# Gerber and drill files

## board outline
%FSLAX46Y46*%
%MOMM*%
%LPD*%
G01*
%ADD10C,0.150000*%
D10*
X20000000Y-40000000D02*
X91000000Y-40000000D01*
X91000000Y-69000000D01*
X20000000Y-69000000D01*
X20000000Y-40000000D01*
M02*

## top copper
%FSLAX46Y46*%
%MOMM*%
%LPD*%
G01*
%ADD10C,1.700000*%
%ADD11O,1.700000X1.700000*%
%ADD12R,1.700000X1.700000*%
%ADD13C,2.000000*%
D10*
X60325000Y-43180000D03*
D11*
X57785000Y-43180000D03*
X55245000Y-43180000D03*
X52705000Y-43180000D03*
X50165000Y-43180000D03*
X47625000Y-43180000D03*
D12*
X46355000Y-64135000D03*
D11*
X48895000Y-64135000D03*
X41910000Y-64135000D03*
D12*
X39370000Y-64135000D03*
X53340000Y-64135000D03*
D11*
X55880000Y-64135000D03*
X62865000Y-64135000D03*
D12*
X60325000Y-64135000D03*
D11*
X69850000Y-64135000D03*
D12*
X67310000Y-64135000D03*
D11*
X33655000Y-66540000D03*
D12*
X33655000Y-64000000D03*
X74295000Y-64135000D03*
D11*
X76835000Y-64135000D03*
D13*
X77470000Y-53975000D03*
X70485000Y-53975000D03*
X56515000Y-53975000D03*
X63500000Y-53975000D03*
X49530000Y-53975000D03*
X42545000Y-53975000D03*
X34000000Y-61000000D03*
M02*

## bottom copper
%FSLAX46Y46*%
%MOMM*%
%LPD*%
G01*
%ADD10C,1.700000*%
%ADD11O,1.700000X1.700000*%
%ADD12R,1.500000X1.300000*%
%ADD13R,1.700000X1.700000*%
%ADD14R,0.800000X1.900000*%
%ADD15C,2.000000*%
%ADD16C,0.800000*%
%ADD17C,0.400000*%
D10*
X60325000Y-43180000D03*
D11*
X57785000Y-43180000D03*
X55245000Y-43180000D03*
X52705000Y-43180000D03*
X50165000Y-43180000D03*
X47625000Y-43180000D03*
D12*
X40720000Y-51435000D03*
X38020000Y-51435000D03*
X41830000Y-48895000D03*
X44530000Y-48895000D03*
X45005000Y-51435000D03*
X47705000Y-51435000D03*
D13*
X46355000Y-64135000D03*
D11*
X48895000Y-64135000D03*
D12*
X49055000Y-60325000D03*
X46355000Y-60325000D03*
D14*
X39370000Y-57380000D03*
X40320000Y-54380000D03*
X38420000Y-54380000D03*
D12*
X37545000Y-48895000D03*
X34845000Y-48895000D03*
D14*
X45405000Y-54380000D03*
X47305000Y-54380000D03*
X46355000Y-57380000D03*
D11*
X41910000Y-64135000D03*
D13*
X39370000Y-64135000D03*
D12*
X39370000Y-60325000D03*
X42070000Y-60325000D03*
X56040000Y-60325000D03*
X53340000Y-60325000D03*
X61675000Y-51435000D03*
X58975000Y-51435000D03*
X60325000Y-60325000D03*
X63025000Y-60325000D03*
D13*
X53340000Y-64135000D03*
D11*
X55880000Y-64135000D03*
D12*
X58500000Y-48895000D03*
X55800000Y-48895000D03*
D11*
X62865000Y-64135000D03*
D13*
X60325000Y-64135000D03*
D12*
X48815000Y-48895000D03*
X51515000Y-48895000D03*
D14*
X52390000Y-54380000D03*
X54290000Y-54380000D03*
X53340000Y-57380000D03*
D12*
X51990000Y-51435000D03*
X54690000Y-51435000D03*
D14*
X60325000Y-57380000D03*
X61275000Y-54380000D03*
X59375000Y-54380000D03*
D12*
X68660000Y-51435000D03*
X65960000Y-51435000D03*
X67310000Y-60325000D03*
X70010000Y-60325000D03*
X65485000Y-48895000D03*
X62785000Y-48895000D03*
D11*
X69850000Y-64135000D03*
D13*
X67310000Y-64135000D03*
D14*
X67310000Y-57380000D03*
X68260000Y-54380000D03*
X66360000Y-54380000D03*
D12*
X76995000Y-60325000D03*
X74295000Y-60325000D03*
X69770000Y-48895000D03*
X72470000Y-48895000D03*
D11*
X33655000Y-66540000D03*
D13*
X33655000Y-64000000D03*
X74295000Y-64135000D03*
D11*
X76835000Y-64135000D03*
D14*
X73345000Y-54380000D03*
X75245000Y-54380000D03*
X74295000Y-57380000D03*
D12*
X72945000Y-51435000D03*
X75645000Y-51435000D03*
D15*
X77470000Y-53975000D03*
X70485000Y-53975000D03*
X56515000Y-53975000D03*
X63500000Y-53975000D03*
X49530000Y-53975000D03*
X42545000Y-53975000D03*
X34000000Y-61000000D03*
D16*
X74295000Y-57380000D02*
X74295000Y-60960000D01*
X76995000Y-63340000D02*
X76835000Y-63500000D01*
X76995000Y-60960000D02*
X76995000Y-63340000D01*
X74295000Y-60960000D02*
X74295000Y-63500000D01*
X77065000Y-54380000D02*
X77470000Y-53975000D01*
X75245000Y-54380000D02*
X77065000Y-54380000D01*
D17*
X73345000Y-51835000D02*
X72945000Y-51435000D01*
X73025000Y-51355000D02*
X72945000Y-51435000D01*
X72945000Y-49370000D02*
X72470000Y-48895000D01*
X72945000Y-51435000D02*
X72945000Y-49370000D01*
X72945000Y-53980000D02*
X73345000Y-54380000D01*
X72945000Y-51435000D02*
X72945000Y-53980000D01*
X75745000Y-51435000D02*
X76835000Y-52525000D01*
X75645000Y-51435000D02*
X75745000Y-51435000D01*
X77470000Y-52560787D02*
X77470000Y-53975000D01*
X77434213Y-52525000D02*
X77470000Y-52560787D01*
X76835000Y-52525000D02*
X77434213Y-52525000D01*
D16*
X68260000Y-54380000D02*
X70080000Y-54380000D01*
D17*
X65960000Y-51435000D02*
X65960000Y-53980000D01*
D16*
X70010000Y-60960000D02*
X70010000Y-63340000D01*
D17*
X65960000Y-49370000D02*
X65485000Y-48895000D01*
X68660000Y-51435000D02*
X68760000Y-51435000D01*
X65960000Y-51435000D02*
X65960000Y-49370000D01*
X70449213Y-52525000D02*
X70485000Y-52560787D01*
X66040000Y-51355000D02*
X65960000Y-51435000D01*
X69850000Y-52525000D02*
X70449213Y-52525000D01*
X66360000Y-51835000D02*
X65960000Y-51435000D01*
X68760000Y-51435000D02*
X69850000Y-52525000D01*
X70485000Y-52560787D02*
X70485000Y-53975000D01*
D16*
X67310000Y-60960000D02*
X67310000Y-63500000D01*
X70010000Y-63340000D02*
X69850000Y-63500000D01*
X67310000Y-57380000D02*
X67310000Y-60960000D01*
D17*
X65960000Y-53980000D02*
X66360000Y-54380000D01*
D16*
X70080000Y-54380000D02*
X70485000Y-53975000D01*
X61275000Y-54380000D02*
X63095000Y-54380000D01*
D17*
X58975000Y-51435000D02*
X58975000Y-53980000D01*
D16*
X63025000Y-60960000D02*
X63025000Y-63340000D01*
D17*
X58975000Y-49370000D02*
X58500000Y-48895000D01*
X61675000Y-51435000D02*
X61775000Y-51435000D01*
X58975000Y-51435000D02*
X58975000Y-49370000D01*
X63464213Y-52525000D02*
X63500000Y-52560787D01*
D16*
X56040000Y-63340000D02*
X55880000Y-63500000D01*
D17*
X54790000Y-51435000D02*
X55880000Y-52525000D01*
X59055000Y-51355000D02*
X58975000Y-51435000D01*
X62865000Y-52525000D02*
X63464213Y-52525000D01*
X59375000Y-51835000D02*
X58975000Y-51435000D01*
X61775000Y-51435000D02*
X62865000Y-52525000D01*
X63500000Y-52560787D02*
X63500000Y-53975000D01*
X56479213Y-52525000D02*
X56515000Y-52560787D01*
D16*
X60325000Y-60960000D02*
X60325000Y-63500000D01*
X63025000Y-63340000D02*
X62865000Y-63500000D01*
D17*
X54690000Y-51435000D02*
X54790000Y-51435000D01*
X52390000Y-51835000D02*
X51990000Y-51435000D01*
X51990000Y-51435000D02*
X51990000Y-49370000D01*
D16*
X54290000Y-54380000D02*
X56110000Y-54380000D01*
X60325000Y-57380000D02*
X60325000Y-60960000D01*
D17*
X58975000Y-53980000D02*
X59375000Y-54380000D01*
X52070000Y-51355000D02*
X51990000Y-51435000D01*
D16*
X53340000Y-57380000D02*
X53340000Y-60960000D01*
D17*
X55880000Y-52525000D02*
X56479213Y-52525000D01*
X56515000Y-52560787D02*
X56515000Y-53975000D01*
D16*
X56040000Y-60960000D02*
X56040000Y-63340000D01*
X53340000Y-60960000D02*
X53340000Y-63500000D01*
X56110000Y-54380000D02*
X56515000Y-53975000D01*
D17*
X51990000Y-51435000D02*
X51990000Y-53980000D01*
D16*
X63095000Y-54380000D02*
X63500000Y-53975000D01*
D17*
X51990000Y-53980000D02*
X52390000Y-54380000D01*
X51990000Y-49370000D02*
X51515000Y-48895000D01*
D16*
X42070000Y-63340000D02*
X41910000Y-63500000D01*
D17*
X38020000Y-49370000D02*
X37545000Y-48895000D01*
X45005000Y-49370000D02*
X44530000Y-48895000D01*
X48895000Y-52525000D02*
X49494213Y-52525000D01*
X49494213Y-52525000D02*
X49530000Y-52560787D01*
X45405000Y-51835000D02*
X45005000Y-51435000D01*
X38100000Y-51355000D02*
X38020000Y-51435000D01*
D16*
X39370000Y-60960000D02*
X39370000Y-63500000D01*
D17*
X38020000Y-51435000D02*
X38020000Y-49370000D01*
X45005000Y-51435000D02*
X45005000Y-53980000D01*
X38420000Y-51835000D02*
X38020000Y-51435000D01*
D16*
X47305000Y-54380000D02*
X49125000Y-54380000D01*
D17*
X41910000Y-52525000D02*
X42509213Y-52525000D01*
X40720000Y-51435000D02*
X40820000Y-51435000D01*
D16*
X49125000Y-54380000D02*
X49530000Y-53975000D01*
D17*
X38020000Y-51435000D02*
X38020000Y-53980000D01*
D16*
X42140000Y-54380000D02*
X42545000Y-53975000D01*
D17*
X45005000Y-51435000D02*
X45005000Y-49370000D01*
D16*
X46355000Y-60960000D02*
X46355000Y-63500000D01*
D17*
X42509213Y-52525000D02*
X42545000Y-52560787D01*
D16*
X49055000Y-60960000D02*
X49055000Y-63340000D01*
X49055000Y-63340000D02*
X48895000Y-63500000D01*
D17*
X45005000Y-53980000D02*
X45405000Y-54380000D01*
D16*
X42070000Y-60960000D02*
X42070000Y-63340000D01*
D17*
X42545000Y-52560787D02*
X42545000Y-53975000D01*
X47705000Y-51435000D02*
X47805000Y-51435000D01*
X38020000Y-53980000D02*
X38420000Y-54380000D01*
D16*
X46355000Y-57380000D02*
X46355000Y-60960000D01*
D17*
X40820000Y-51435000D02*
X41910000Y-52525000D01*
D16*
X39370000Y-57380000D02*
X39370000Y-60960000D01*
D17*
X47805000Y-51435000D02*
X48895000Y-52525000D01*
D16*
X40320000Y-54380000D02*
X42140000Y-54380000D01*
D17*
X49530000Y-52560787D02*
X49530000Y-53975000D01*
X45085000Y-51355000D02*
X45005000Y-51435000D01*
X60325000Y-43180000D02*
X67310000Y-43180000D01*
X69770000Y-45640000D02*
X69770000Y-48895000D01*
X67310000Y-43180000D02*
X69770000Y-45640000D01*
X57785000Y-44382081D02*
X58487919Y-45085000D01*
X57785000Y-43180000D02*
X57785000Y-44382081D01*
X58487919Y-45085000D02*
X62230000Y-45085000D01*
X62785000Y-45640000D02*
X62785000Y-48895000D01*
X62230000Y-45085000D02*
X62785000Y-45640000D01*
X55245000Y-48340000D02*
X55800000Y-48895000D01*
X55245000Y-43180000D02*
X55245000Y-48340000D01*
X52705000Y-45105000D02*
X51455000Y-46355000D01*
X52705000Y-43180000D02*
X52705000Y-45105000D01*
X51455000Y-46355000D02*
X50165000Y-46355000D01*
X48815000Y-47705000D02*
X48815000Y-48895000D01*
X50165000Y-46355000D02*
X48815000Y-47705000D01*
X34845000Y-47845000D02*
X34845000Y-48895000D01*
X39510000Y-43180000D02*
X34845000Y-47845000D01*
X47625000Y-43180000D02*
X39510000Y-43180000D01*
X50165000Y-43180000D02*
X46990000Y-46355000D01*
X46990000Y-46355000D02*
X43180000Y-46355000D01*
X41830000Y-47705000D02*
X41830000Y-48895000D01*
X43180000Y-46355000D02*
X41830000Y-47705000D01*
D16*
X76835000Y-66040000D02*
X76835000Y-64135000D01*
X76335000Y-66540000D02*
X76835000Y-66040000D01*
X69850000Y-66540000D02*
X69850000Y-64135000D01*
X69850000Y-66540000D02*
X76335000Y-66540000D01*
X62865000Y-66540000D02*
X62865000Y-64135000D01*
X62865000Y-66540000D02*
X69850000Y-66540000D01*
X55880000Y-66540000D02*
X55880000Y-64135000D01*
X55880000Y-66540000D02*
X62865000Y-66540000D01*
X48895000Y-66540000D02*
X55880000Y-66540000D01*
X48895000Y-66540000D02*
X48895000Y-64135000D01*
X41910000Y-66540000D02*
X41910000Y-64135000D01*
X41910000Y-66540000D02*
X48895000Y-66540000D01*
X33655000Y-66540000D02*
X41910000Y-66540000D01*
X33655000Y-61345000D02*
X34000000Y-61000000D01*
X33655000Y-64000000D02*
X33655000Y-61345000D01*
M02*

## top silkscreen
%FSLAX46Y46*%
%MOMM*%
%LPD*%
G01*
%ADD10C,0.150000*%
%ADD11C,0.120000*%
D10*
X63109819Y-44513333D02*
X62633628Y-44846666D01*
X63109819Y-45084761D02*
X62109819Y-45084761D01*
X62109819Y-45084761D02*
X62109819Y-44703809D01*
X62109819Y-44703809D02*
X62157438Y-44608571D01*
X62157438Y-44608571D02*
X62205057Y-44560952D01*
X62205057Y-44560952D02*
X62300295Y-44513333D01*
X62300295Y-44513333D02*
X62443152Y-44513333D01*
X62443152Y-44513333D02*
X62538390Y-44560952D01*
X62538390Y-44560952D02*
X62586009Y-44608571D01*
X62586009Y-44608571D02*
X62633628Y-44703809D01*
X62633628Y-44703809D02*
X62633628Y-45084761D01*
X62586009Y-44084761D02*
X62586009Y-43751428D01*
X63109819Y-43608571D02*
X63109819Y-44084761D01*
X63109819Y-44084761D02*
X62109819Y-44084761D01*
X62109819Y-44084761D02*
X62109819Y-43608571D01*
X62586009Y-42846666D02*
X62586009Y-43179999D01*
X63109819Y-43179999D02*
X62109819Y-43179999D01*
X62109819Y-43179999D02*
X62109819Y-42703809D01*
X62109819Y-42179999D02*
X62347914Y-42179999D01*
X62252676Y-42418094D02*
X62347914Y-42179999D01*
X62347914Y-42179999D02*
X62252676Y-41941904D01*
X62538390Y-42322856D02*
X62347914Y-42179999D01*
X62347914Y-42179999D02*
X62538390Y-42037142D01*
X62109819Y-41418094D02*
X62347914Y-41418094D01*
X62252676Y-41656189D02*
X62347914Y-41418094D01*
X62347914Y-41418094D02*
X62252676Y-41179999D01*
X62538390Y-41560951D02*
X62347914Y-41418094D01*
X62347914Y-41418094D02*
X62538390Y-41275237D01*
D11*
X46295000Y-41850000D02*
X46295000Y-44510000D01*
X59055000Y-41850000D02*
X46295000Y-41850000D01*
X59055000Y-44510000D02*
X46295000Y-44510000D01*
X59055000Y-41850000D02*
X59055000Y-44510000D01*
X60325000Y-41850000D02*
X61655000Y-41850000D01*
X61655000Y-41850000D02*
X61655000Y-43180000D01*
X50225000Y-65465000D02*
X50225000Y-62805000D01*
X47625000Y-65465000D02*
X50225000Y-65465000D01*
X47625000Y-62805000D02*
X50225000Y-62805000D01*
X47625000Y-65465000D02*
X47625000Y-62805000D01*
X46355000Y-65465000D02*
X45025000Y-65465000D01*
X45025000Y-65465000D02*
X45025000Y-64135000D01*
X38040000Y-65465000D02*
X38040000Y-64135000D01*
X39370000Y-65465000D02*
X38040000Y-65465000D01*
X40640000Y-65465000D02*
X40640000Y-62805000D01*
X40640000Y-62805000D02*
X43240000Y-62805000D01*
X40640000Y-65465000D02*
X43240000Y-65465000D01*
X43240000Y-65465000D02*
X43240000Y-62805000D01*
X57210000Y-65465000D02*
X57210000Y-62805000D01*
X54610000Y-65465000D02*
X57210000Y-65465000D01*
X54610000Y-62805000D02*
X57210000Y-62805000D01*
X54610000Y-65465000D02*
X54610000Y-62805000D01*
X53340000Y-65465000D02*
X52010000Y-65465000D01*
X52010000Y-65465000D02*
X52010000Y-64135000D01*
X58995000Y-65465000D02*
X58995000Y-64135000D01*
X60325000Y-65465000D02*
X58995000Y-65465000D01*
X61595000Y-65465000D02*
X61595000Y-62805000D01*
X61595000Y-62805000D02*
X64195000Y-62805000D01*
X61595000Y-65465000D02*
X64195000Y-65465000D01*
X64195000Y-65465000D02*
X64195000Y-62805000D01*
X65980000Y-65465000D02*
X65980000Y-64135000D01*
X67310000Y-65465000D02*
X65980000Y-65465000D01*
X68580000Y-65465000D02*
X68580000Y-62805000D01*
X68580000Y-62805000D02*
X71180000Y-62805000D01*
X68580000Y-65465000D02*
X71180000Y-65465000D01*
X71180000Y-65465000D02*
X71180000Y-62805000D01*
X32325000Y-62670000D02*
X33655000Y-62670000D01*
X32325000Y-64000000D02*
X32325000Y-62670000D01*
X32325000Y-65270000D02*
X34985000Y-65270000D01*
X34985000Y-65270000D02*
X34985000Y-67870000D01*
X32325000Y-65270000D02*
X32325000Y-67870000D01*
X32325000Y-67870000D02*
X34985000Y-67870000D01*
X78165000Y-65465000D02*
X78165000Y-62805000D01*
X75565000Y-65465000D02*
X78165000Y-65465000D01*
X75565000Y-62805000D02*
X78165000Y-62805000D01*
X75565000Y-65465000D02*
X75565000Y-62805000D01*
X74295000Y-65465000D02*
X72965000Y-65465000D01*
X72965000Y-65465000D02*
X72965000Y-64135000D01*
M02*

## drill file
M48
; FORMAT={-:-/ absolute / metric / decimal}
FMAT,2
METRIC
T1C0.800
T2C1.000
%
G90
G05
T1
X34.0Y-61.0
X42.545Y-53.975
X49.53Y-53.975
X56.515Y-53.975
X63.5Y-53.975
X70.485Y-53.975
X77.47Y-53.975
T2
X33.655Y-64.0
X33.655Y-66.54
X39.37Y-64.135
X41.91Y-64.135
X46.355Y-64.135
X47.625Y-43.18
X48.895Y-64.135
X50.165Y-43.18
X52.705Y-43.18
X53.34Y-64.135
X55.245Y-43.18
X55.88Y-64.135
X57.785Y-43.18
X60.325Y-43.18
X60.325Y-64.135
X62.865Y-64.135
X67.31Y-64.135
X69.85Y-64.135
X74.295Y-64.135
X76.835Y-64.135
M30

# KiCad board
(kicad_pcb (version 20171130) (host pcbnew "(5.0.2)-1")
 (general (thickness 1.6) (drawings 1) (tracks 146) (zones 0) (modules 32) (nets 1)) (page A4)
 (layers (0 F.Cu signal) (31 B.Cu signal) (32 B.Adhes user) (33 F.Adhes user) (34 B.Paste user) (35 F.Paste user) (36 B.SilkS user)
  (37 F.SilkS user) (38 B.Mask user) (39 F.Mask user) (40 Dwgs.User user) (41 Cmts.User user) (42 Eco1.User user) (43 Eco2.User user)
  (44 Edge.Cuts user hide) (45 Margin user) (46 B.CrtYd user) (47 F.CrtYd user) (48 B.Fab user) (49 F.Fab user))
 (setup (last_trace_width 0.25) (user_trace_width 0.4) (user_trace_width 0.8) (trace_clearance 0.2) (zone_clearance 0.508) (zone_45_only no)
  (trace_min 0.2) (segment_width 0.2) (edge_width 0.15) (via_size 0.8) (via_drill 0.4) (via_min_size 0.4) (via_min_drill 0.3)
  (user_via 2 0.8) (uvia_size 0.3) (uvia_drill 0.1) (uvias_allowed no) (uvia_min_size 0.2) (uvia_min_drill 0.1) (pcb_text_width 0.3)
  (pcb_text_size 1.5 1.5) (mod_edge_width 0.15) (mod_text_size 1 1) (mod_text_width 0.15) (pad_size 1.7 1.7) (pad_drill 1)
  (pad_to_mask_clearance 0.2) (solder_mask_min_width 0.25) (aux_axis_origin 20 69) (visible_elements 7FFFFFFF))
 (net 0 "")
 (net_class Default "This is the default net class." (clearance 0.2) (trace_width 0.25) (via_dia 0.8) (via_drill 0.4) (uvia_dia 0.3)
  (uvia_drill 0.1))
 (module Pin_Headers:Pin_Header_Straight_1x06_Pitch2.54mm (layer F.Cu) (at 60.325 43.18 270)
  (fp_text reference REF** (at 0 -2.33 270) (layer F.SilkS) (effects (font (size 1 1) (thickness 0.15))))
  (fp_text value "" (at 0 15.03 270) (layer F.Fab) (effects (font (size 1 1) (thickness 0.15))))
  (fp_line (start -1.33 14.03) (end 1.33 14.03) (layer F.SilkS) (width 0.12))
  (fp_line (start -1.33 1.27) (end -1.33 14.03) (layer F.SilkS) (width 0.12))
  (fp_line (start 1.33 1.27) (end 1.33 14.03) (layer F.SilkS) (width 0.12))
  (fp_line (start -1.33 1.27) (end 1.33 1.27) (layer F.SilkS) (width 0.12))
  (fp_line (start -1.33 0) (end -1.33 -1.33) (layer F.SilkS) (width 0.12))
  (fp_line (start -1.33 -1.33) (end 0 -1.33) (layer F.SilkS) (width 0.12))
  (pad 1 thru_hole circle (at 0 0 270) (size 1.7 1.7) (drill 1) (layers *.Cu *.Mask))
  (pad 2 thru_hole oval (at 0 2.54 270) (size 1.7 1.7) (drill 1) (layers *.Cu *.Mask))
  (pad 3 thru_hole oval (at 0 5.08 270) (size 1.7 1.7) (drill 1) (layers *.Cu *.Mask))
  (pad 4 thru_hole oval (at 0 7.62 270) (size 1.7 1.7) (drill 1) (layers *.Cu *.Mask))
  (pad 5 thru_hole oval (at 0 10.16 270) (size 1.7 1.7) (drill 1) (layers *.Cu *.Mask))
  (pad 6 thru_hole oval (at 0 12.7 270) (size 1.7 1.7) (drill 1) (layers *.Cu *.Mask)))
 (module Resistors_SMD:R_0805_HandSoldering (layer B.Cu) (at 39.37 51.435)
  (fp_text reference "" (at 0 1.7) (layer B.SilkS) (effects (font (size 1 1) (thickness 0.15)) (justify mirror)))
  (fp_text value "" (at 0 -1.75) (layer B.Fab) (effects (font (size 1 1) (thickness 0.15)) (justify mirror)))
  (pad 2 smd rect (at 1.35 0) (size 1.5 1.3) (layers B.Cu B.Paste B.Mask))
  (pad 1 smd rect (at -1.35 0) (size 1.5 1.3) (layers B.Cu B.Paste B.Mask)))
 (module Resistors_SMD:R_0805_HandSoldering (layer B.Cu) (at 43.18 48.895 180)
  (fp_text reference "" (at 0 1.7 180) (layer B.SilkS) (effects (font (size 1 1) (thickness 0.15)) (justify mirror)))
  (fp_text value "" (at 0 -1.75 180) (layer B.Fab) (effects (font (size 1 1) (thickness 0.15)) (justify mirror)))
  (pad 2 smd rect (at 1.35 0 180) (size 1.5 1.3) (layers B.Cu B.Paste B.Mask))
  (pad 1 smd rect (at -1.35 0 180) (size 1.5 1.3) (layers B.Cu B.Paste B.Mask)))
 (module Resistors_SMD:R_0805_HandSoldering (layer B.Cu) (at 46.355 51.435)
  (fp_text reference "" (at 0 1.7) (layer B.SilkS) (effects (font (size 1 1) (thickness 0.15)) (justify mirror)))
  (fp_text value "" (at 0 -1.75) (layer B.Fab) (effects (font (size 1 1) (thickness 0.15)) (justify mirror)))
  (pad 1 smd rect (at -1.35 0) (size 1.5 1.3) (layers B.Cu B.Paste B.Mask))
  (pad 2 smd rect (at 1.35 0) (size 1.5 1.3) (layers B.Cu B.Paste B.Mask)))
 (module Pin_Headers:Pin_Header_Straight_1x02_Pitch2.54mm (layer F.Cu) (at 46.355 64.135 90)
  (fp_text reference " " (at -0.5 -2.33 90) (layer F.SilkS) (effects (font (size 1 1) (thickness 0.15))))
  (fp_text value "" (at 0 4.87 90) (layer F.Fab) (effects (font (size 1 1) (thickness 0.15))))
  (fp_line (start -1.33 3.87) (end 1.33 3.87) (layer F.SilkS) (width 0.12))
  (fp_line (start -1.33 1.27) (end -1.33 3.87) (layer F.SilkS) (width 0.12))
  (fp_line (start 1.33 1.27) (end 1.33 3.87) (layer F.SilkS) (width 0.12))
  (fp_line (start -1.33 1.27) (end 1.33 1.27) (layer F.SilkS) (width 0.12))
  (fp_line (start -1.33 0) (end -1.33 -1.33) (layer F.SilkS) (width 0.12))
  (fp_line (start -1.33 -1.33) (end 0 -1.33) (layer F.SilkS) (width 0.12))
  (pad 1 thru_hole rect (at 0 0 90) (size 1.7 1.7) (drill 1) (layers *.Cu *.Mask))
  (pad 2 thru_hole oval (at 0 2.54 90) (size 1.7 1.7) (drill 1) (layers *.Cu *.Mask)))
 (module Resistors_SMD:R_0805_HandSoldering (layer B.Cu) (at 47.705 60.325 180)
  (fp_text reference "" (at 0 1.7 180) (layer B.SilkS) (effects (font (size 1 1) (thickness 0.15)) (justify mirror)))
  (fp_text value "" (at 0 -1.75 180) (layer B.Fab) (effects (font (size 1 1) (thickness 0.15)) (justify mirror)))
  (pad 1 smd rect (at -1.35 0 180) (size 1.5 1.3) (layers B.Cu B.Paste B.Mask))
  (pad 2 smd rect (at 1.35 0 180) (size 1.5 1.3) (layers B.Cu B.Paste B.Mask)))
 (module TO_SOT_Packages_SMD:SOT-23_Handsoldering (layer B.Cu) (at 39.37 55.88 270)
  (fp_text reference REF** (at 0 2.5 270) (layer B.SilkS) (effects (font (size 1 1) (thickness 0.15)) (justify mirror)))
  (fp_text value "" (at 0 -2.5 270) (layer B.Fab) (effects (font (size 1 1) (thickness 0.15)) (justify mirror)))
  (pad D smd rect (at 1.5 0 270) (size 1.9 0.8) (layers B.Cu B.Paste B.Mask))
  (pad S smd rect (at -1.5 -0.95 270) (size 1.9 0.8) (layers B.Cu B.Paste B.Mask))
  (pad G smd rect (at -1.5 0.95 270) (size 1.9 0.8) (layers B.Cu B.Paste B.Mask)))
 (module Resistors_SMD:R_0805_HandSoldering (layer B.Cu) (at 36.195 48.895 180)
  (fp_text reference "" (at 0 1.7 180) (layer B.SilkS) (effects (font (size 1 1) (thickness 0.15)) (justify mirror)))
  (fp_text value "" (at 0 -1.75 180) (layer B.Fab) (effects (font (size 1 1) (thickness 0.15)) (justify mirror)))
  (pad 1 smd rect (at -1.35 0 180) (size 1.5 1.3) (layers B.Cu B.Paste B.Mask))
  (pad 2 smd rect (at 1.35 0 180) (size 1.5 1.3) (layers B.Cu B.Paste B.Mask)))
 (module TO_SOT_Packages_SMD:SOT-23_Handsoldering (layer B.Cu) (at 46.355 55.88 270)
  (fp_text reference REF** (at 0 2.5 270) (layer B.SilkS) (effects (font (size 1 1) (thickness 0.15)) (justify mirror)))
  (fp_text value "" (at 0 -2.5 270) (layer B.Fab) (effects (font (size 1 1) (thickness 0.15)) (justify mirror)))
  (pad G smd rect (at -1.5 0.95 270) (size 1.9 0.8) (layers B.Cu B.Paste B.Mask))
  (pad S smd rect (at -1.5 -0.95 270) (size 1.9 0.8) (layers B.Cu B.Paste B.Mask))
  (pad D smd rect (at 1.5 0 270) (size 1.9 0.8) (layers B.Cu B.Paste B.Mask)))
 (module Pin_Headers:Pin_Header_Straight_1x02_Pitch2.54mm (layer F.Cu) (at 39.37 64.135 90)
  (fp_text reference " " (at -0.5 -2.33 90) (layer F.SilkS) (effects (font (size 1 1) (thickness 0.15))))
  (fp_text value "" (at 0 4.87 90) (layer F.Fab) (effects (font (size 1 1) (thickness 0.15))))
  (fp_line (start -1.33 -1.33) (end 0 -1.33) (layer F.SilkS) (width 0.12))
  (fp_line (start -1.33 0) (end -1.33 -1.33) (layer F.SilkS) (width 0.12))
  (fp_line (start -1.33 1.27) (end 1.33 1.27) (layer F.SilkS) (width 0.12))
  (fp_line (start 1.33 1.27) (end 1.33 3.87) (layer F.SilkS) (width 0.12))
  (fp_line (start -1.33 1.27) (end -1.33 3.87) (layer F.SilkS) (width 0.12))
  (fp_line (start -1.33 3.87) (end 1.33 3.87) (layer F.SilkS) (width 0.12))
  (pad 2 thru_hole oval (at 0 2.54 90) (size 1.7 1.7) (drill 1) (layers *.Cu *.Mask))
  (pad 1 thru_hole rect (at 0 0 90) (size 1.7 1.7) (drill 1) (layers *.Cu *.Mask)))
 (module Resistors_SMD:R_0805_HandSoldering (layer B.Cu) (at 40.72 60.325 180)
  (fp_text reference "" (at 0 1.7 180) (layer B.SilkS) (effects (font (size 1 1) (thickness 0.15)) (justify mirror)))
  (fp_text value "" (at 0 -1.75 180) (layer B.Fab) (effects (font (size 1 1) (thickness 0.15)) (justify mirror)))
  (pad 2 smd rect (at 1.35 0 180) (size 1.5 1.3) (layers B.Cu B.Paste B.Mask))
  (pad 1 smd rect (at -1.35 0 180) (size 1.5 1.3) (layers B.Cu B.Paste B.Mask)))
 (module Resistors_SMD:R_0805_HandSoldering (layer B.Cu) (at 54.69 60.325 180)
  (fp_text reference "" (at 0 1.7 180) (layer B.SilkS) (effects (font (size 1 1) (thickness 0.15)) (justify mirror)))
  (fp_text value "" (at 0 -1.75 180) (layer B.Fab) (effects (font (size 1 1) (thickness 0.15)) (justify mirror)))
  (pad 1 smd rect (at -1.35 0 180) (size 1.5 1.3) (layers B.Cu B.Paste B.Mask))
  (pad 2 smd rect (at 1.35 0 180) (size 1.5 1.3) (layers B.Cu B.Paste B.Mask)))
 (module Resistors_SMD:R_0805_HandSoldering (layer B.Cu) (at 60.325 51.435)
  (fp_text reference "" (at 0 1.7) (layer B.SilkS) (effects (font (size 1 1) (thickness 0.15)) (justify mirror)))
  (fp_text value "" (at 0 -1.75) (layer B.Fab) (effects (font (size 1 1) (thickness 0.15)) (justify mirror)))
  (pad 2 smd rect (at 1.35 0) (size 1.5 1.3) (layers B.Cu B.Paste B.Mask))
  (pad 1 smd rect (at -1.35 0) (size 1.5 1.3) (layers B.Cu B.Paste B.Mask)))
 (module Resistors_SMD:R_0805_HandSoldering (layer B.Cu) (at 61.675 60.325 180)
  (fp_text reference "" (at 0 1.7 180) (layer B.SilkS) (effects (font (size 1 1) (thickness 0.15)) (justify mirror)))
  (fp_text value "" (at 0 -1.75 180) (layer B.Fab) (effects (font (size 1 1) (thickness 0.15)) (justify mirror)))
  (pad 2 smd rect (at 1.35 0 180) (size 1.5 1.3) (layers B.Cu B.Paste B.Mask))
  (pad 1 smd rect (at -1.35 0 180) (size 1.5 1.3) (layers B.Cu B.Paste B.Mask)))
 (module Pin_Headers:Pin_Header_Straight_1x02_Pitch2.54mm (layer F.Cu) (at 53.34 64.135 90)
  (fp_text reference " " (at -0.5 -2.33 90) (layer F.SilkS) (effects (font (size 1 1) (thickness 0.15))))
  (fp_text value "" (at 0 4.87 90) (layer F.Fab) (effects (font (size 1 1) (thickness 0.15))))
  (fp_line (start -1.33 3.87) (end 1.33 3.87) (layer F.SilkS) (width 0.12))
  (fp_line (start -1.33 1.27) (end -1.33 3.87) (layer F.SilkS) (width 0.12))
  (fp_line (start 1.33 1.27) (end 1.33 3.87) (layer F.SilkS) (width 0.12))
  (fp_line (start -1.33 1.27) (end 1.33 1.27) (layer F.SilkS) (width 0.12))
  (fp_line (start -1.33 0) (end -1.33 -1.33) (layer F.SilkS) (width 0.12))
  (fp_line (start -1.33 -1.33) (end 0 -1.33) (layer F.SilkS) (width 0.12))
  (pad 1 thru_hole rect (at 0 0 90) (size 1.7 1.7) (drill 1) (layers *.Cu *.Mask))
  (pad 2 thru_hole oval (at 0 2.54 90) (size 1.7 1.7) (drill 1) (layers *.Cu *.Mask)))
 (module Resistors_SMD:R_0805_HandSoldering (layer B.Cu) (at 57.15 48.895 180)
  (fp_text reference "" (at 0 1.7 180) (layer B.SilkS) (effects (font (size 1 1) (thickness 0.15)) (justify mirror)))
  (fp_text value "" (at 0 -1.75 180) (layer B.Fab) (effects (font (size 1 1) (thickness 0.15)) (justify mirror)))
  (pad 1 smd rect (at -1.35 0 180) (size 1.5 1.3) (layers B.Cu B.Paste B.Mask))
  (pad 2 smd rect (at 1.35 0 180) (size 1.5 1.3) (layers B.Cu B.Paste B.Mask)))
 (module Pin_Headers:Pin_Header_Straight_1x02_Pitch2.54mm (layer F.Cu) (at 60.325 64.135 90)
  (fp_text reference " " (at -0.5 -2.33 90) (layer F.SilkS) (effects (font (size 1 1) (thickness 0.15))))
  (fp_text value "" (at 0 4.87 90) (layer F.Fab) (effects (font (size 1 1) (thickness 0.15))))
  (fp_line (start -1.33 -1.33) (end 0 -1.33) (layer F.SilkS) (width 0.12))
  (fp_line (start -1.33 0) (end -1.33 -1.33) (layer F.SilkS) (width 0.12))
  (fp_line (start -1.33 1.27) (end 1.33 1.27) (layer F.SilkS) (width 0.12))
  (fp_line (start 1.33 1.27) (end 1.33 3.87) (layer F.SilkS) (width 0.12))
  (fp_line (start -1.33 1.27) (end -1.33 3.87) (layer F.SilkS) (width 0.12))
  (fp_line (start -1.33 3.87) (end 1.33 3.87) (layer F.SilkS) (width 0.12))
  (pad 2 thru_hole oval (at 0 2.54 90) (size 1.7 1.7) (drill 1) (layers *.Cu *.Mask))
  (pad 1 thru_hole rect (at 0 0 90) (size 1.7 1.7) (drill 1) (layers *.Cu *.Mask)))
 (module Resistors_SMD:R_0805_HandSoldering (layer B.Cu) (at 50.165 48.895 180)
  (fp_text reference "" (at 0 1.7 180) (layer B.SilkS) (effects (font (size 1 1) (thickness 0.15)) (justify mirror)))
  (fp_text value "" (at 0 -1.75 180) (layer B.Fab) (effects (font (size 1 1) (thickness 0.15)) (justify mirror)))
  (pad 2 smd rect (at 1.35 0 180) (size 1.5 1.3) (layers B.Cu B.Paste B.Mask))
  (pad 1 smd rect (at -1.35 0 180) (size 1.5 1.3) (layers B.Cu B.Paste B.Mask)))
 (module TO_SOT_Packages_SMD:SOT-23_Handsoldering (layer B.Cu) (at 53.34 55.88 270)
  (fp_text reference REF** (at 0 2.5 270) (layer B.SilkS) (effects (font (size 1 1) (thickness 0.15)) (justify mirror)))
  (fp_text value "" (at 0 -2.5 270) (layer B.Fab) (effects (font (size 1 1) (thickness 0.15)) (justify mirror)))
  (pad G smd rect (at -1.5 0.95 270) (size 1.9 0.8) (layers B.Cu B.Paste B.Mask))
  (pad S smd rect (at -1.5 -0.95 270) (size 1.9 0.8) (layers B.Cu B.Paste B.Mask))
  (pad D smd rect (at 1.5 0 270) (size 1.9 0.8) (layers B.Cu B.Paste B.Mask)))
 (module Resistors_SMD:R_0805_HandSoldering (layer B.Cu) (at 53.34 51.435)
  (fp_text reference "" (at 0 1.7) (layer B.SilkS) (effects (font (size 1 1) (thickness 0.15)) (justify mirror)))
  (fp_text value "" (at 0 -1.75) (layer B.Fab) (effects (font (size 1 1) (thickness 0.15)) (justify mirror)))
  (pad 1 smd rect (at -1.35 0) (size 1.5 1.3) (layers B.Cu B.Paste B.Mask))
  (pad 2 smd rect (at 1.35 0) (size 1.5 1.3) (layers B.Cu B.Paste B.Mask)))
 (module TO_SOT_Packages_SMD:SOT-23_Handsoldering (layer B.Cu) (at 60.325 55.88 270)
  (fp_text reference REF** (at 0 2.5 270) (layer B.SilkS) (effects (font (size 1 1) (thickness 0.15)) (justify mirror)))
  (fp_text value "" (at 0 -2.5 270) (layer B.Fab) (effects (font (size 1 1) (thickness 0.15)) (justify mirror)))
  (pad D smd rect (at 1.5 0 270) (size 1.9 0.8) (layers B.Cu B.Paste B.Mask))
  (pad S smd rect (at -1.5 -0.95 270) (size 1.9 0.8) (layers B.Cu B.Paste B.Mask))
  (pad G smd rect (at -1.5 0.95 270) (size 1.9 0.8) (layers B.Cu B.Paste B.Mask)))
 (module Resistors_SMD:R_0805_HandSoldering (layer B.Cu) (at 67.31 51.435)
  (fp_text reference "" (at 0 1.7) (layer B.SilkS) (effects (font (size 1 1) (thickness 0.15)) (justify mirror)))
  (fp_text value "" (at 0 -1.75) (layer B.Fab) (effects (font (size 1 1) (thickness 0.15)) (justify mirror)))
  (pad 2 smd rect (at 1.35 0) (size 1.5 1.3) (layers B.Cu B.Paste B.Mask))
  (pad 1 smd rect (at -1.35 0) (size 1.5 1.3) (layers B.Cu B.Paste B.Mask)))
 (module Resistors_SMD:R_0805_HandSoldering (layer B.Cu) (at 68.66 60.325 180)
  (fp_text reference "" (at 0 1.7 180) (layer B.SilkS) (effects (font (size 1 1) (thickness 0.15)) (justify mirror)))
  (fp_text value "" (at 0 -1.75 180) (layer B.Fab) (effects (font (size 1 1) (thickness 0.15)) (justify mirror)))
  (pad 2 smd rect (at 1.35 0 180) (size 1.5 1.3) (layers B.Cu B.Paste B.Mask))
  (pad 1 smd rect (at -1.35 0 180) (size 1.5 1.3) (layers B.Cu B.Paste B.Mask)))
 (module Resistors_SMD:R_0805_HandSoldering (layer B.Cu) (at 64.135 48.895 180)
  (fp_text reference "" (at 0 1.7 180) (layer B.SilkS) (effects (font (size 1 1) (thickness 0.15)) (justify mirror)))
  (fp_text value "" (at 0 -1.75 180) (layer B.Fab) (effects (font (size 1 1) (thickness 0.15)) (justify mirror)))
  (pad 1 smd rect (at -1.35 0 180) (size 1.5 1.3) (layers B.Cu B.Paste B.Mask))
  (pad 2 smd rect (at 1.35 0 180) (size 1.5 1.3) (layers B.Cu B.Paste B.Mask)))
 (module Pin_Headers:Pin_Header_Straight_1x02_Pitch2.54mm (layer F.Cu) (at 67.31 64.135 90)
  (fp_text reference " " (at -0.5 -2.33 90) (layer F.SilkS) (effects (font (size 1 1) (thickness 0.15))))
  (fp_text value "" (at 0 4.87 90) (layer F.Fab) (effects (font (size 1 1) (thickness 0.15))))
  (fp_line (start -1.33 -1.33) (end 0 -1.33) (layer F.SilkS) (width 0.12))
  (fp_line (start -1.33 0) (end -1.33 -1.33) (layer F.SilkS) (width 0.12))
  (fp_line (start -1.33 1.27) (end 1.33 1.27) (layer F.SilkS) (width 0.12))
  (fp_line (start 1.33 1.27) (end 1.33 3.87) (layer F.SilkS) (width 0.12))
  (fp_line (start -1.33 1.27) (end -1.33 3.87) (layer F.SilkS) (width 0.12))
  (fp_line (start -1.33 3.87) (end 1.33 3.87) (layer F.SilkS) (width 0.12))
  (pad 2 thru_hole oval (at 0 2.54 90) (size 1.7 1.7) (drill 1) (layers *.Cu *.Mask))
  (pad 1 thru_hole rect (at 0 0 90) (size 1.7 1.7) (drill 1) (layers *.Cu *.Mask)))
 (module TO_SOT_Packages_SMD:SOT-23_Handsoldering (layer B.Cu) (at 67.31 55.88 270)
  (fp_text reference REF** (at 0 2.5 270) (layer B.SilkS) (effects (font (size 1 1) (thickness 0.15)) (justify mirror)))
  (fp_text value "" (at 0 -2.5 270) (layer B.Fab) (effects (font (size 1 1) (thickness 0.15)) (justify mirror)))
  (pad D smd rect (at 1.5 0 270) (size 1.9 0.8) (layers B.Cu B.Paste B.Mask))
  (pad S smd rect (at -1.5 -0.95 270) (size 1.9 0.8) (layers B.Cu B.Paste B.Mask))
  (pad G smd rect (at -1.5 0.95 270) (size 1.9 0.8) (layers B.Cu B.Paste B.Mask)))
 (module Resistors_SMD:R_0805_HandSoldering (layer B.Cu) (at 75.645 60.325 180)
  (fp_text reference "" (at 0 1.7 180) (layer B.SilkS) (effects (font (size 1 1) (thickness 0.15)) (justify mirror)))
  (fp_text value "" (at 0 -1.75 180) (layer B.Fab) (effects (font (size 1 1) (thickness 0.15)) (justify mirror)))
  (pad 1 smd rect (at -1.35 0 180) (size 1.5 1.3) (layers B.Cu B.Paste B.Mask))
  (pad 2 smd rect (at 1.35 0 180) (size 1.5 1.3) (layers B.Cu B.Paste B.Mask)))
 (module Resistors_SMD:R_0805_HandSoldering (layer B.Cu) (at 71.12 48.895 180)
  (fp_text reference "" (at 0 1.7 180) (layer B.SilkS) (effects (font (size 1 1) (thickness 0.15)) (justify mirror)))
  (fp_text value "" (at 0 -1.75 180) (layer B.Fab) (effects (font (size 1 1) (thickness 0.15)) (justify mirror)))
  (pad 2 smd rect (at 1.35 0 180) (size 1.5 1.3) (layers B.Cu B.Paste B.Mask))
  (pad 1 smd rect (at -1.35 0 180) (size 1.5 1.3) (layers B.Cu B.Paste B.Mask)))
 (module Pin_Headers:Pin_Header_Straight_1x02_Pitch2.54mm (layer F.Cu) (at 33.655 64)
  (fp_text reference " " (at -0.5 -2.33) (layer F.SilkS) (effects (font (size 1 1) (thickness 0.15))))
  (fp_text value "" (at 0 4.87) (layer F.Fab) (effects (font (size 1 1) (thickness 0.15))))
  (fp_line (start -1.33 -1.33) (end 0 -1.33) (layer F.SilkS) (width 0.12))
  (fp_line (start -1.33 0) (end -1.33 -1.33) (layer F.SilkS) (width 0.12))
  (fp_line (start -1.33 1.27) (end 1.33 1.27) (layer F.SilkS) (width 0.12))
  (fp_line (start 1.33 1.27) (end 1.33 3.87) (layer F.SilkS) (width 0.12))
  (fp_line (start -1.33 1.27) (end -1.33 3.87) (layer F.SilkS) (width 0.12))
  (fp_line (start -1.33 3.87) (end 1.33 3.87) (layer F.SilkS) (width 0.12))
  (pad 2 thru_hole oval (at 0 2.54) (size 1.7 1.7) (drill 1) (layers *.Cu *.Mask))
  (pad 1 thru_hole rect (at 0 0) (size 1.7 1.7) (drill 1) (layers *.Cu *.Mask)))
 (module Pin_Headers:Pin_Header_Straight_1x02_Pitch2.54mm (layer F.Cu) (at 74.295 64.135 90)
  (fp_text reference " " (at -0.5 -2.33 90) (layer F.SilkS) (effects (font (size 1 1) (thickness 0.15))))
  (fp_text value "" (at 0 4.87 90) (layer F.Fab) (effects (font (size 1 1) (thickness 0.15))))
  (fp_line (start -1.33 3.87) (end 1.33 3.87) (layer F.SilkS) (width 0.12))
  (fp_line (start -1.33 1.27) (end -1.33 3.87) (layer F.SilkS) (width 0.12))
  (fp_line (start 1.33 1.27) (end 1.33 3.87) (layer F.SilkS) (width 0.12))
  (fp_line (start -1.33 1.27) (end 1.33 1.27) (layer F.SilkS) (width 0.12))
  (fp_line (start -1.33 0) (end -1.33 -1.33) (layer F.SilkS) (width 0.12))
  (fp_line (start -1.33 -1.33) (end 0 -1.33) (layer F.SilkS) (width 0.12))
  (pad 1 thru_hole rect (at 0 0 90) (size 1.7 1.7) (drill 1) (layers *.Cu *.Mask))
  (pad 2 thru_hole oval (at 0 2.54 90) (size 1.7 1.7) (drill 1) (layers *.Cu *.Mask)))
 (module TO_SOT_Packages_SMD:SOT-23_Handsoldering (layer B.Cu) (at 74.295 55.88 270)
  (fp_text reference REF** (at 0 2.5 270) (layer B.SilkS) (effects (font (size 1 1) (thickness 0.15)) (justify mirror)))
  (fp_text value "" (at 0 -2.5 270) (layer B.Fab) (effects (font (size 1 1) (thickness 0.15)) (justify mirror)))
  (pad G smd rect (at -1.5 0.95 270) (size 1.9 0.8) (layers B.Cu B.Paste B.Mask))
  (pad S smd rect (at -1.5 -0.95 270) (size 1.9 0.8) (layers B.Cu B.Paste B.Mask))
  (pad D smd rect (at 1.5 0 270) (size 1.9 0.8) (layers B.Cu B.Paste B.Mask)))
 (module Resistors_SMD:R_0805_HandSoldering (layer B.Cu) (at 74.295 51.435)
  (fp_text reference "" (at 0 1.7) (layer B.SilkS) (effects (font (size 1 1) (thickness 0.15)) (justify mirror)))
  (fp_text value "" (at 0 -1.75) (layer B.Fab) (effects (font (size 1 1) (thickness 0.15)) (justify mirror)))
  (pad 1 smd rect (at -1.35 0) (size 1.5 1.3) (layers B.Cu B.Paste B.Mask))
  (pad 2 smd rect (at 1.35 0) (size 1.5 1.3) (layers B.Cu B.Paste B.Mask)))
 (gr_poly (pts (xy 20 40) (xy 91 40) (xy 91 69) (xy 20 69)) (layer Edge.Cuts) (width 0.15))
 (segment (start 74.295 57.38) (end 74.295 60.96) (width 0.8) (layer B.Cu) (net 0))
 (segment (start 76.995 63.34) (end 76.835 63.5) (width 0.8) (layer B.Cu) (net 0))
 (segment (start 76.995 60.96) (end 76.995 63.34) (width 0.8) (layer B.Cu) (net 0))
 (segment (start 74.295 60.96) (end 74.295 63.5) (width 0.8) (layer B.Cu) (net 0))
 (via (at 77.47 53.975) (size 2) (drill 0.8) (layers F.Cu B.Cu) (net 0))
 (segment (start 77.065 54.38) (end 77.47 53.975) (width 0.8) (layer B.Cu) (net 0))
 (segment (start 75.245 54.38) (end 77.065 54.38) (width 0.8) (layer B.Cu) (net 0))
 (segment (start 73.345 51.835) (end 72.945 51.435) (width 0.4) (layer B.Cu) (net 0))
 (segment (start 73.025 51.355) (end 72.945 51.435) (width 0.4) (layer B.Cu) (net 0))
 (segment (start 72.945 49.37) (end 72.47 48.895) (width 0.4) (layer B.Cu) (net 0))
 (segment (start 72.945 51.435) (end 72.945 49.37) (width 0.4) (layer B.Cu) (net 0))
 (segment (start 72.945 53.98) (end 73.345 54.38) (width 0.4) (layer B.Cu) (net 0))
 (segment (start 72.945 51.435) (end 72.945 53.98) (width 0.4) (layer B.Cu) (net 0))
 (segment (start 75.745 51.435) (end 76.835 52.525) (width 0.4) (layer B.Cu) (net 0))
 (segment (start 75.645 51.435) (end 75.745 51.435) (width 0.4) (layer B.Cu) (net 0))
 (segment (start 77.47 52.560787) (end 77.47 53.975) (width 0.4) (layer B.Cu) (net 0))
 (segment (start 77.434213 52.525) (end 77.47 52.560787) (width 0.4) (layer B.Cu) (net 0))
 (segment (start 76.835 52.525) (end 77.434213 52.525) (width 0.4) (layer B.Cu) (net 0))
 (segment (start 68.26 54.38) (end 70.08 54.38) (width 0.8) (layer B.Cu) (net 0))
 (segment (start 65.96 51.435) (end 65.96 53.98) (width 0.4) (layer B.Cu) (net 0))
 (segment (start 70.01 60.96) (end 70.01 63.34) (width 0.8) (layer B.Cu) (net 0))
 (segment (start 65.96 49.37) (end 65.485 48.895) (width 0.4) (layer B.Cu) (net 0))
 (segment (start 68.66 51.435) (end 68.76 51.435) (width 0.4) (layer B.Cu) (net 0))
 (segment (start 65.96 51.435) (end 65.96 49.37) (width 0.4) (layer B.Cu) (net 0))
 (segment (start 70.449213 52.525) (end 70.485 52.560787) (width 0.4) (layer B.Cu) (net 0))
 (segment (start 66.04 51.355) (end 65.96 51.435) (width 0.4) (layer B.Cu) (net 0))
 (segment (start 69.85 52.525) (end 70.449213 52.525) (width 0.4) (layer B.Cu) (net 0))
 (segment (start 66.36 51.835) (end 65.96 51.435) (width 0.4) (layer B.Cu) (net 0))
 (segment (start 68.76 51.435) (end 69.85 52.525) (width 0.4) (layer B.Cu) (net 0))
 (segment (start 70.485 52.560787) (end 70.485 53.975) (width 0.4) (layer B.Cu) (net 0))
 (segment (start 67.31 60.96) (end 67.31 63.5) (width 0.8) (layer B.Cu) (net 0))
 (segment (start 70.01 63.34) (end 69.85 63.5) (width 0.8) (layer B.Cu) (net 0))
 (segment (start 67.31 57.38) (end 67.31 60.96) (width 0.8) (layer B.Cu) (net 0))
 (segment (start 65.96 53.98) (end 66.36 54.38) (width 0.4) (layer B.Cu) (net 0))
 (via (at 70.485 53.975) (size 2) (drill 0.8) (layers F.Cu B.Cu) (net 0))
 (segment (start 70.08 54.38) (end 70.485 53.975) (width 0.8) (layer B.Cu) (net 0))
 (segment (start 61.275 54.38) (end 63.095 54.38) (width 0.8) (layer B.Cu) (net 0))
 (segment (start 58.975 51.435) (end 58.975 53.98) (width 0.4) (layer B.Cu) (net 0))
 (segment (start 63.025 60.96) (end 63.025 63.34) (width 0.8) (layer B.Cu) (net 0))
 (segment (start 58.975 49.37) (end 58.5 48.895) (width 0.4) (layer B.Cu) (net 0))
 (segment (start 61.675 51.435) (end 61.775 51.435) (width 0.4) (layer B.Cu) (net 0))
 (segment (start 58.975 51.435) (end 58.975 49.37) (width 0.4) (layer B.Cu) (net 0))
 (segment (start 63.464213 52.525) (end 63.5 52.560787) (width 0.4) (layer B.Cu) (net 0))
 (segment (start 56.04 63.34) (end 55.88 63.5) (width 0.8) (layer B.Cu) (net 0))
 (segment (start 54.79 51.435) (end 55.88 52.525) (width 0.4) (layer B.Cu) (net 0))
 (segment (start 59.055 51.355) (end 58.975 51.435) (width 0.4) (layer B.Cu) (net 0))
 (segment (start 62.865 52.525) (end 63.464213 52.525) (width 0.4) (layer B.Cu) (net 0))
 (segment (start 59.375 51.835) (end 58.975 51.435) (width 0.4) (layer B.Cu) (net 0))
 (segment (start 61.775 51.435) (end 62.865 52.525) (width 0.4) (layer B.Cu) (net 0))
 (segment (start 63.5 52.560787) (end 63.5 53.975) (width 0.4) (layer B.Cu) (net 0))
 (segment (start 56.479213 52.525) (end 56.515 52.560787) (width 0.4) (layer B.Cu) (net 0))
 (segment (start 60.325 60.96) (end 60.325 63.5) (width 0.8) (layer B.Cu) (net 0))
 (segment (start 63.025 63.34) (end 62.865 63.5) (width 0.8) (layer B.Cu) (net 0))
 (via (at 56.515 53.975) (size 2) (drill 0.8) (layers F.Cu B.Cu) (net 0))
 (segment (start 54.69 51.435) (end 54.79 51.435) (width 0.4) (layer B.Cu) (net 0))
 (segment (start 52.39 51.835) (end 51.99 51.435) (width 0.4) (layer B.Cu) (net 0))
 (segment (start 51.99 51.435) (end 51.99 49.37) (width 0.4) (layer B.Cu) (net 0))
 (segment (start 54.29 54.38) (end 56.11 54.38) (width 0.8) (layer B.Cu) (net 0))
 (segment (start 60.325 57.38) (end 60.325 60.96) (width 0.8) (layer B.Cu) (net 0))
 (segment (start 58.975 53.98) (end 59.375 54.38) (width 0.4) (layer B.Cu) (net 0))
 (via (at 63.5 53.975) (size 2) (drill 0.8) (layers F.Cu B.Cu) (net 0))
 (segment (start 52.07 51.355) (end 51.99 51.435) (width 0.4) (layer B.Cu) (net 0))
 (segment (start 53.34 57.38) (end 53.34 60.96) (width 0.8) (layer B.Cu) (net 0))
 (segment (start 55.88 52.525) (end 56.479213 52.525) (width 0.4) (layer B.Cu) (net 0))
 (segment (start 56.515 52.560787) (end 56.515 53.975) (width 0.4) (layer B.Cu) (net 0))
 (segment (start 56.04 60.96) (end 56.04 63.34) (width 0.8) (layer B.Cu) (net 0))
 (segment (start 53.34 60.96) (end 53.34 63.5) (width 0.8) (layer B.Cu) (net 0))
 (segment (start 56.11 54.38) (end 56.515 53.975) (width 0.8) (layer B.Cu) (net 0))
 (segment (start 51.99 51.435) (end 51.99 53.98) (width 0.4) (layer B.Cu) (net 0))
 (segment (start 63.095 54.38) (end 63.5 53.975) (width 0.8) (layer B.Cu) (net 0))
 (segment (start 51.99 53.98) (end 52.39 54.38) (width 0.4) (layer B.Cu) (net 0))
 (segment (start 51.99 49.37) (end 51.515 48.895) (width 0.4) (layer B.Cu) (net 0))
 (segment (start 42.07 63.34) (end 41.91 63.5) (width 0.8) (layer B.Cu) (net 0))
 (segment (start 38.02 49.37) (end 37.545 48.895) (width 0.4) (layer B.Cu) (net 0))
 (segment (start 45.005 49.37) (end 44.53 48.895) (width 0.4) (layer B.Cu) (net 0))
 (segment (start 48.895 52.525) (end 49.494213 52.525) (width 0.4) (layer B.Cu) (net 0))
 (segment (start 49.494213 52.525) (end 49.53 52.560787) (width 0.4) (layer B.Cu) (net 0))
 (segment (start 45.405 51.835) (end 45.005 51.435) (width 0.4) (layer B.Cu) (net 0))
 (segment (start 38.1 51.355) (end 38.02 51.435) (width 0.4) (layer B.Cu) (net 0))
 (via (at 49.53 53.975) (size 2) (drill 0.8) (layers F.Cu B.Cu) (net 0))
 (segment (start 39.37 60.96) (end 39.37 63.5) (width 0.8) (layer B.Cu) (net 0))
 (segment (start 38.02 51.435) (end 38.02 49.37) (width 0.4) (layer B.Cu) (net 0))
 (segment (start 45.005 51.435) (end 45.005 53.98) (width 0.4) (layer B.Cu) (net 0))
 (segment (start 38.42 51.835) (end 38.02 51.435) (width 0.4) (layer B.Cu) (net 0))
 (segment (start 47.305 54.38) (end 49.125 54.38) (width 0.8) (layer B.Cu) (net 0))
 (segment (start 41.91 52.525) (end 42.509213 52.525) (width 0.4) (layer B.Cu) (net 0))
 (segment (start 40.72 51.435) (end 40.82 51.435) (width 0.4) (layer B.Cu) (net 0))
 (segment (start 49.125 54.38) (end 49.53 53.975) (width 0.8) (layer B.Cu) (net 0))
 (segment (start 38.02 51.435) (end 38.02 53.98) (width 0.4) (layer B.Cu) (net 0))
 (segment (start 42.14 54.38) (end 42.545 53.975) (width 0.8) (layer B.Cu) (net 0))
 (segment (start 45.005 51.435) (end 45.005 49.37) (width 0.4) (layer B.Cu) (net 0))
 (segment (start 46.355 60.96) (end 46.355 63.5) (width 0.8) (layer B.Cu) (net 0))
 (segment (start 42.509213 52.525) (end 42.545 52.560787) (width 0.4) (layer B.Cu) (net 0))
 (segment (start 49.055 60.96) (end 49.055 63.34) (width 0.8) (layer B.Cu) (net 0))
 (via (at 42.545 53.975) (size 2) (drill 0.8) (layers F.Cu B.Cu) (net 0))
 (segment (start 49.055 63.34) (end 48.895 63.5) (width 0.8) (layer B.Cu) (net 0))
 (segment (start 45.005 53.98) (end 45.405 54.38) (width 0.4) (layer B.Cu) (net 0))
 (segment (start 42.07 60.96) (end 42.07 63.34) (width 0.8) (layer B.Cu) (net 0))
 (segment (start 42.545 52.560787) (end 42.545 53.975) (width 0.4) (layer B.Cu) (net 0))
 (segment (start 47.705 51.435) (end 47.805 51.435) (width 0.4) (layer B.Cu) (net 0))
 (segment (start 38.02 53.98) (end 38.42 54.38) (width 0.4) (layer B.Cu) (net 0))
 (segment (start 46.355 57.38) (end 46.355 60.96) (width 0.8) (layer B.Cu) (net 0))
 (segment (start 40.82 51.435) (end 41.91 52.525) (width 0.4) (layer B.Cu) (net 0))
 (segment (start 39.37 57.38) (end 39.37 60.96) (width 0.8) (layer B.Cu) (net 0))
 (segment (start 47.805 51.435) (end 48.895 52.525) (width 0.4) (layer B.Cu) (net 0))
 (segment (start 40.32 54.38) (end 42.14 54.38) (width 0.8) (layer B.Cu) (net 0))
 (segment (start 49.53 52.560787) (end 49.53 53.975) (width 0.4) (layer B.Cu) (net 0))
 (segment (start 45.085 51.355) (end 45.005 51.435) (width 0.4) (layer B.Cu) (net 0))
 (segment (start 60.325 43.18) (end 67.31 43.18) (width 0.4) (layer B.Cu) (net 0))
 (segment (start 69.77 45.64) (end 69.77 48.895) (width 0.4) (layer B.Cu) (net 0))
 (segment (start 67.31 43.18) (end 69.77 45.64) (width 0.4) (layer B.Cu) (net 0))
 (segment (start 57.785 44.382081) (end 58.487919 45.085) (width 0.4) (layer B.Cu) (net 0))
 (segment (start 57.785 43.18) (end 57.785 44.382081) (width 0.4) (layer B.Cu) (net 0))
 (segment (start 58.487919 45.085) (end 62.23 45.085) (width 0.4) (layer B.Cu) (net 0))
 (segment (start 62.785 45.64) (end 62.785 48.895) (width 0.4) (layer B.Cu) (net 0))
 (segment (start 62.23 45.085) (end 62.785 45.64) (width 0.4) (layer B.Cu) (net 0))
 (segment (start 55.245 48.34) (end 55.8 48.895) (width 0.4) (layer B.Cu) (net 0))
 (segment (start 55.245 43.18) (end 55.245 48.34) (width 0.4) (layer B.Cu) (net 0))
 (segment (start 52.705 45.105) (end 51.455 46.355) (width 0.4) (layer B.Cu) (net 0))
 (segment (start 52.705 43.18) (end 52.705 45.105) (width 0.4) (layer B.Cu) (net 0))
 (segment (start 51.455 46.355) (end 50.165 46.355) (width 0.4) (layer B.Cu) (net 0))
 (segment (start 48.815 47.705) (end 48.815 48.895) (width 0.4) (layer B.Cu) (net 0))
 (segment (start 50.165 46.355) (end 48.815 47.705) (width 0.4) (layer B.Cu) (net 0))
 (segment (start 34.845 47.845) (end 34.845 48.895) (width 0.4) (layer B.Cu) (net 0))
 (segment (start 39.51 43.18) (end 34.845 47.845) (width 0.4) (layer B.Cu) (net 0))
 (segment (start 47.625 43.18) (end 39.51 43.18) (width 0.4) (layer B.Cu) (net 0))
 (segment (start 50.165 43.18) (end 46.99 46.355) (width 0.4) (layer B.Cu) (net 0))
 (segment (start 46.99 46.355) (end 43.18 46.355) (width 0.4) (layer B.Cu) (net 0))
 (segment (start 41.83 47.705) (end 41.83 48.895) (width 0.4) (layer B.Cu) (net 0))
 (segment (start 43.18 46.355) (end 41.83 47.705) (width 0.4) (layer B.Cu) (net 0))
 (segment (start 76.835 66.04) (end 76.835 64.135) (width 0.8) (layer B.Cu) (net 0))
 (segment (start 76.335 66.54) (end 76.835 66.04) (width 0.8) (layer B.Cu) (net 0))
 (segment (start 69.85 66.54) (end 69.85 64.135) (width 0.8) (layer B.Cu) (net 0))
 (segment (start 69.85 66.54) (end 76.335 66.54) (width 0.8) (layer B.Cu) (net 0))
 (segment (start 62.865 66.54) (end 62.865 64.135) (width 0.8) (layer B.Cu) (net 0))
 (segment (start 62.865 66.54) (end 69.85 66.54) (width 0.8) (layer B.Cu) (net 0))
 (segment (start 55.88 66.54) (end 55.88 64.135) (width 0.8) (layer B.Cu) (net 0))
 (segment (start 55.88 66.54) (end 62.865 66.54) (width 0.8) (layer B.Cu) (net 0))
 (segment (start 48.895 66.54) (end 55.88 66.54) (width 0.8) (layer B.Cu) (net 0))
 (segment (start 48.895 66.54) (end 48.895 64.135) (width 0.8) (layer B.Cu) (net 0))
 (segment (start 41.91 66.54) (end 41.91 64.135) (width 0.8) (layer B.Cu) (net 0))
 (segment (start 41.91 66.54) (end 48.895 66.54) (width 0.8) (layer B.Cu) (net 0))
 (segment (start 33.655 66.54) (end 41.91 66.54) (width 0.8) (layer B.Cu) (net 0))
 (via (at 34 61) (size 2) (drill 0.8) (layers F.Cu B.Cu) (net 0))
 (segment (start 33.655 61.345) (end 34 61) (width 0.8) (layer B.Cu) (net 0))
 (segment (start 33.655 64) (end 33.655 61.345) (width 0.8) (layer B.Cu) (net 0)))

